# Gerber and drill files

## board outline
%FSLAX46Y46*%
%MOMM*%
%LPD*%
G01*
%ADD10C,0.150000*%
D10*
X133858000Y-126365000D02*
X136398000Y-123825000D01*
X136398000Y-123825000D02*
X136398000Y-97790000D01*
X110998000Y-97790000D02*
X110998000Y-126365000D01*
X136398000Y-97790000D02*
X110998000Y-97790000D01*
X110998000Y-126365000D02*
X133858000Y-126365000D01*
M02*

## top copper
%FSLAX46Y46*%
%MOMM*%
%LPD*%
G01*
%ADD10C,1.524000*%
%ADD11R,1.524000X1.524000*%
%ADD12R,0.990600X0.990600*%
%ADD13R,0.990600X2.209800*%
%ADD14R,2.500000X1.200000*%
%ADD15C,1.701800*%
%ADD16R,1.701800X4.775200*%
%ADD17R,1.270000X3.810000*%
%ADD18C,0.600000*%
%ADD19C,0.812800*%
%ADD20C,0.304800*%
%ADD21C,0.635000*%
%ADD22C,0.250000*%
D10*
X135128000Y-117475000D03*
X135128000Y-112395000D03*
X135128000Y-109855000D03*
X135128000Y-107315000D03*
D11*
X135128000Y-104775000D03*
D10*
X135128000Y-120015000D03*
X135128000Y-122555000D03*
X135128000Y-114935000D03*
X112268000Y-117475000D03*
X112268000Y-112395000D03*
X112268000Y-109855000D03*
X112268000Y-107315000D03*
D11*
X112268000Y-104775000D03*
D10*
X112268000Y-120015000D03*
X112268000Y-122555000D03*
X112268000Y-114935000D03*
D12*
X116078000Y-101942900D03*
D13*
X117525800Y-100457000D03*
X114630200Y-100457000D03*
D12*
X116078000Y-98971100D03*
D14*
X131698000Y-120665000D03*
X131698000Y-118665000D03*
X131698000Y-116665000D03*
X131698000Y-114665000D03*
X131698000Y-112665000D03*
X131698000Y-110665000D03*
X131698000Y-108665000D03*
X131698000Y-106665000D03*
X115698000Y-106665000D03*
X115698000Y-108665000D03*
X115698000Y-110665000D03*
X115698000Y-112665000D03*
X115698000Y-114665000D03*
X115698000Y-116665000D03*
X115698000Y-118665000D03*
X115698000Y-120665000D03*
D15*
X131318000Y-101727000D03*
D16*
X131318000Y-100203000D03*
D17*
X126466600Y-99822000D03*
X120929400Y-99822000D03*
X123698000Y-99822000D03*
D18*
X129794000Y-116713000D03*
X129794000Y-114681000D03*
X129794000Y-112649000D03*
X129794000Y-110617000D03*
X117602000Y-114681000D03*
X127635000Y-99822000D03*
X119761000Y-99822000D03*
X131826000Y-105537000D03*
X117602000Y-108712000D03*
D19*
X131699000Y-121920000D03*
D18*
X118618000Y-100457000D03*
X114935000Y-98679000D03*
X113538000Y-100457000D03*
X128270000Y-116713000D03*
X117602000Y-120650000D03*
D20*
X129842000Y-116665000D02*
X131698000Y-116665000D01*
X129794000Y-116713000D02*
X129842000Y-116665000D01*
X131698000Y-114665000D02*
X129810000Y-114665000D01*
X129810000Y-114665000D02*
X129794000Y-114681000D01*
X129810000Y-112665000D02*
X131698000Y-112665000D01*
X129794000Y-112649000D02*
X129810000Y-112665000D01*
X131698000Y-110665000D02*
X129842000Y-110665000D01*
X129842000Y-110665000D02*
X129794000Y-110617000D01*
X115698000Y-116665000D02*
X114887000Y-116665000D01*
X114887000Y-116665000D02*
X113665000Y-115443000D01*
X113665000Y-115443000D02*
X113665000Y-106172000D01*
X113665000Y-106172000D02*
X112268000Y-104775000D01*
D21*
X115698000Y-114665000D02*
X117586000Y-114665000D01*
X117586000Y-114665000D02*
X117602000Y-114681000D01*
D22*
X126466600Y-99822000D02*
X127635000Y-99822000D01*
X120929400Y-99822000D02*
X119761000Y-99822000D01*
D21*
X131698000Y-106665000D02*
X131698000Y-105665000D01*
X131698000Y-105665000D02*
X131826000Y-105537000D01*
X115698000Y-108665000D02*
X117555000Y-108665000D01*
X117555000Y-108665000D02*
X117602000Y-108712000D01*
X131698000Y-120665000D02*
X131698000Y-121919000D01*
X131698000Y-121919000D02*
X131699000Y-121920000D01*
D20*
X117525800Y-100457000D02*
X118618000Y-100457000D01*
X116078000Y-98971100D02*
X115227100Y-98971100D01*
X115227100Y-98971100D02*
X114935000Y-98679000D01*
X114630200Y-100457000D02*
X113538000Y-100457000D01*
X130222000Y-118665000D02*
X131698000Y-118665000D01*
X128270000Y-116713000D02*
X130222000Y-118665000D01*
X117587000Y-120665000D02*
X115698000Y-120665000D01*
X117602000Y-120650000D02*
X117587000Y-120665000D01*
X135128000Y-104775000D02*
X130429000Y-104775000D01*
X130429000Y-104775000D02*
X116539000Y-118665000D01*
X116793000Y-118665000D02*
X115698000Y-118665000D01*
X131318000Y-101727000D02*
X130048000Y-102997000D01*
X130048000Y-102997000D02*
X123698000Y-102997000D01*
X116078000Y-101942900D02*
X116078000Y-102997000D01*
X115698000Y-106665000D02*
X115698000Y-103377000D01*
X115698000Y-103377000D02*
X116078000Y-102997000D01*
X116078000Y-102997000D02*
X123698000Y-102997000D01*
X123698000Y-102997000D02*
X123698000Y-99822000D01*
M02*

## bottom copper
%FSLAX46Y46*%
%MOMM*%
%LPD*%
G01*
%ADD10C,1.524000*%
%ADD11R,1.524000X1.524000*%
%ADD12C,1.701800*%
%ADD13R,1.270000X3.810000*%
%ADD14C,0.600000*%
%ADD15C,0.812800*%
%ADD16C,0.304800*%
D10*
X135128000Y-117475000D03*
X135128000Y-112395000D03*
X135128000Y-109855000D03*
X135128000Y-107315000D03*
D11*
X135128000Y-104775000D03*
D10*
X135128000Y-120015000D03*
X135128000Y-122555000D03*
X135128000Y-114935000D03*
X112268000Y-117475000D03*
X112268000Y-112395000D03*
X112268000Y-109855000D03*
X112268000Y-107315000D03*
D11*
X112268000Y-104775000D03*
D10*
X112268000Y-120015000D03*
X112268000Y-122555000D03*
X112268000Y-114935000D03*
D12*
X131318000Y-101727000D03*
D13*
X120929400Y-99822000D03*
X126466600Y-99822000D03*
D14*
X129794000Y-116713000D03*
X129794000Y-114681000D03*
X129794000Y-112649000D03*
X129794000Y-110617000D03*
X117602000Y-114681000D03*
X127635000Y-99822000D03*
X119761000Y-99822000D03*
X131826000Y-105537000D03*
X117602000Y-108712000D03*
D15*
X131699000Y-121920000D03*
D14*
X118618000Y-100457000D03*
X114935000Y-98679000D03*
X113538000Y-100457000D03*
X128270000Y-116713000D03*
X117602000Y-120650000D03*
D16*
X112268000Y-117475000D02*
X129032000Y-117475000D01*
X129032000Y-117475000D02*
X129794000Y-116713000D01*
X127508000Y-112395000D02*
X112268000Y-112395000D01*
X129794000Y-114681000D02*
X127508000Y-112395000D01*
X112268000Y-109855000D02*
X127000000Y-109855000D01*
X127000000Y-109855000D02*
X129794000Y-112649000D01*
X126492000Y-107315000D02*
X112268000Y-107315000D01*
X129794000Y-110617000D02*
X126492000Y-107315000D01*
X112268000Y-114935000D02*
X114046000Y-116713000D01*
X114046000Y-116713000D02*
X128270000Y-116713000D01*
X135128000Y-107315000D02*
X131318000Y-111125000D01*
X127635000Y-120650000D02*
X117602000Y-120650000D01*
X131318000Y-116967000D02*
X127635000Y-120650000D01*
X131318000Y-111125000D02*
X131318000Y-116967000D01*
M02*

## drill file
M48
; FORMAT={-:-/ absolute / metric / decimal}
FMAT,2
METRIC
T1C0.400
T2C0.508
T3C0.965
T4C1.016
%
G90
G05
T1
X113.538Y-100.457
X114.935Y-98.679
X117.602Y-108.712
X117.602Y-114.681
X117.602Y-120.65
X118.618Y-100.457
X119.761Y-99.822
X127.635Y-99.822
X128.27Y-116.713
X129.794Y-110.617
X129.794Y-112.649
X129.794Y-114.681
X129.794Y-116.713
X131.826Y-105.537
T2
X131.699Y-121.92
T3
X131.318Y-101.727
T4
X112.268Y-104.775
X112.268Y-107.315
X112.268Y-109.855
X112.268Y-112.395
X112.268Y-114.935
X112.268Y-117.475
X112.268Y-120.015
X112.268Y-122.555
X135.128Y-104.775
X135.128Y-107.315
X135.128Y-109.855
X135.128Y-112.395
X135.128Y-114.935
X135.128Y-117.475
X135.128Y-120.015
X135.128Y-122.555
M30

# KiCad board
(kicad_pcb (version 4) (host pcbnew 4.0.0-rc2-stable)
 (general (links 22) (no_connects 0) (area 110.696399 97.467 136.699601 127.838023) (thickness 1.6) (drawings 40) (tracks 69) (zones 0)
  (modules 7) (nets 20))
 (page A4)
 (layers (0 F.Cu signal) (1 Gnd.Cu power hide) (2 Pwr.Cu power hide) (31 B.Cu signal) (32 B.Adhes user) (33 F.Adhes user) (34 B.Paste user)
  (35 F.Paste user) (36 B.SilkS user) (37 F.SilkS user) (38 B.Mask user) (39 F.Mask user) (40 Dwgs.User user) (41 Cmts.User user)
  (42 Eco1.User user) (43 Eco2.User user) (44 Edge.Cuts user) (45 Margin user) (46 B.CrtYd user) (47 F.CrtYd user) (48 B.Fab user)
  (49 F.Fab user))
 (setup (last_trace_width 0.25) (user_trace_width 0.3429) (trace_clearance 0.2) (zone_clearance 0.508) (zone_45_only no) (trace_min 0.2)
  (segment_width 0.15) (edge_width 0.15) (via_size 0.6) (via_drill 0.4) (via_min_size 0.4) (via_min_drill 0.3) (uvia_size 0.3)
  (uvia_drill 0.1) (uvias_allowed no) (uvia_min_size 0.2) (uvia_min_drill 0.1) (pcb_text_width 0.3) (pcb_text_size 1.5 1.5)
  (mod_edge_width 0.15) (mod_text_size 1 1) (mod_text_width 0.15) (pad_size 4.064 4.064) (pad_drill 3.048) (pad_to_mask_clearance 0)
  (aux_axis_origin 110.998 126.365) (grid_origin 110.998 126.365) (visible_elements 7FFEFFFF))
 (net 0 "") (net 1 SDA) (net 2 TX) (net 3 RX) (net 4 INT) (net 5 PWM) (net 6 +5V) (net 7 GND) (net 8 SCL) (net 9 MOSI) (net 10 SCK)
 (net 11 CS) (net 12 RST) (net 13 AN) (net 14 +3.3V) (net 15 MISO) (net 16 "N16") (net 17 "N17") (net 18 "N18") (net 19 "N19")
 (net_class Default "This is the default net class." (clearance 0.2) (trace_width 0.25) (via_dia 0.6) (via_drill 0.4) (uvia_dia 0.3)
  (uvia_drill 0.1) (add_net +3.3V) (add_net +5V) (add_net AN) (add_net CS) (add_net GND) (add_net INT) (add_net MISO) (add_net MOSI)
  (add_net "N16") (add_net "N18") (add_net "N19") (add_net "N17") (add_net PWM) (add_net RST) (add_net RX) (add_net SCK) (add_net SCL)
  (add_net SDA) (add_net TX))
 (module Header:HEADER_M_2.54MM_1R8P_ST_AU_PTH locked (layer B.Cu) (at 135.128 113.665 270)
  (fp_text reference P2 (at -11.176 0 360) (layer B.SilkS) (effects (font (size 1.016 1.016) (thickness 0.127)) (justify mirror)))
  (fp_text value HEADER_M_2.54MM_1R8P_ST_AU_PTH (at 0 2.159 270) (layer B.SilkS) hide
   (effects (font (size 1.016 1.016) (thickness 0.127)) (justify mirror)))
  (pad 6 thru_hole circle (at 3.81 0 270) (size 1.524 1.524) (drill 1.016) (layers *.Cu *.Mask) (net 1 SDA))
  (pad 4 thru_hole circle (at -1.27 0 270) (size 1.524 1.524) (drill 1.016) (layers *.Cu *.Mask) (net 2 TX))
  (pad 3 thru_hole circle (at -3.81 0 270) (size 1.524 1.524) (drill 1.016) (layers *.Cu *.Mask) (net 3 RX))
  (pad 2 thru_hole circle (at -6.35 0 270) (size 1.524 1.524) (drill 1.016) (layers *.Cu *.Mask) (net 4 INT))
  (pad 1 thru_hole rect (at -8.89 0 270) (size 1.524 1.524) (drill 1.016) (layers *.Cu *.Mask) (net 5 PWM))
  (pad 7 thru_hole circle (at 6.35 0 270) (size 1.524 1.524) (drill 1.016) (layers *.Cu *.Mask) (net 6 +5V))
  (pad 8 thru_hole circle (at 8.89 0 270) (size 1.524 1.524) (drill 1.016) (layers *.Cu *.Mask) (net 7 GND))
  (pad 5 thru_hole circle (at 1.27 0 270) (size 1.524 1.524) (drill 1.016) (layers *.Cu *.Mask) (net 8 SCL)))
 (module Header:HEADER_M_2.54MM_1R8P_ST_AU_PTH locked (layer B.Cu) (at 112.268 113.665 270)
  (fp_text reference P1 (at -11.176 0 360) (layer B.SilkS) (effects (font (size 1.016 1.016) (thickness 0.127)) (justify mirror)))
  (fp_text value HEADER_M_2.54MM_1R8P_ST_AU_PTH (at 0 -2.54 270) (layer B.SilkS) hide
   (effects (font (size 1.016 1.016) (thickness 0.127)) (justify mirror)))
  (pad 6 thru_hole circle (at 3.81 0 270) (size 1.524 1.524) (drill 1.016) (layers *.Cu *.Mask) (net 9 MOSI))
  (pad 4 thru_hole circle (at -1.27 0 270) (size 1.524 1.524) (drill 1.016) (layers *.Cu *.Mask) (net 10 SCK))
  (pad 3 thru_hole circle (at -3.81 0 270) (size 1.524 1.524) (drill 1.016) (layers *.Cu *.Mask) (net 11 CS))
  (pad 2 thru_hole circle (at -6.35 0 270) (size 1.524 1.524) (drill 1.016) (layers *.Cu *.Mask) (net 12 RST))
  (pad 1 thru_hole rect (at -8.89 0 270) (size 1.524 1.524) (drill 1.016) (layers *.Cu *.Mask) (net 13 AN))
  (pad 7 thru_hole circle (at 6.35 0 270) (size 1.524 1.524) (drill 1.016) (layers *.Cu *.Mask) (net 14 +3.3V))
  (pad 8 thru_hole circle (at 8.89 0 270) (size 1.524 1.524) (drill 1.016) (layers *.Cu *.Mask) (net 7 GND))
  (pad 5 thru_hole circle (at 1.27 0 270) (size 1.524 1.524) (drill 1.016) (layers *.Cu *.Mask) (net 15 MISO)))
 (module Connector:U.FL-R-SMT (layer F.Cu) (at 116.078 100.457)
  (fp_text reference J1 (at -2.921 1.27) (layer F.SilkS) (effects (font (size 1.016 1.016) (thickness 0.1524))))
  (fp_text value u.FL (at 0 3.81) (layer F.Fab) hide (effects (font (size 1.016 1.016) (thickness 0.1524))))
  (pad 1 smd rect (at 0 1.4859) (size 0.9906 0.9906) (layers F.Cu F.Paste F.Mask) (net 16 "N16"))
  (pad 4 smd rect (at 1.4478 0) (size 0.9906 2.2098) (layers F.Cu F.Paste F.Mask) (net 7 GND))
  (pad 2 smd rect (at -1.4478 0) (size 0.9906 2.2098) (layers F.Cu F.Paste F.Mask) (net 7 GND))
  (pad 3 smd rect (at 0 -1.4859) (size 0.9906 0.9906) (layers F.Cu F.Paste F.Mask) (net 7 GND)))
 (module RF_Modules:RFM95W (layer F.Cu) (at 123.698 113.665 180)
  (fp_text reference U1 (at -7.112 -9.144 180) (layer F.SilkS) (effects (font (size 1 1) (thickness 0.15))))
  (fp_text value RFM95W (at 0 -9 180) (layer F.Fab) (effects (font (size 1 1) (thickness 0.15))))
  (pad 1 smd rect (at -8 -7 180) (size 2.5 1.2) (layers F.Cu F.Paste F.Mask) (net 7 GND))
  (pad 2 smd rect (at -8 -5 180) (size 2.5 1.2) (layers F.Cu F.Paste F.Mask) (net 15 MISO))
  (pad 3 smd rect (at -8 -3 180) (size 2.5 1.2) (layers F.Cu F.Paste F.Mask) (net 9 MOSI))
  (pad 4 smd rect (at -8 -1 180) (size 2.5 1.2) (layers F.Cu F.Paste F.Mask) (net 10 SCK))
  (pad 5 smd rect (at -8 1 180) (size 2.5 1.2) (layers F.Cu F.Paste F.Mask) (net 11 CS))
  (pad 6 smd rect (at -8 3 180) (size 2.5 1.2) (layers F.Cu F.Paste F.Mask) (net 12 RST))
  (pad 7 smd rect (at -8 5 180) (size 2.5 1.2) (layers F.Cu F.Paste F.Mask) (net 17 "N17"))
  (pad 8 smd rect (at -8 7 180) (size 2.5 1.2) (layers F.Cu F.Paste F.Mask) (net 7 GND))
  (pad 9 smd rect (at 8 7 180) (size 2.5 1.2) (layers F.Cu F.Paste F.Mask) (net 16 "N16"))
  (pad 10 smd rect (at 8 5 180) (size 2.5 1.2) (layers F.Cu F.Paste F.Mask) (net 7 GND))
  (pad 11 smd rect (at 8 3 180) (size 2.5 1.2) (layers F.Cu F.Paste F.Mask) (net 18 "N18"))
  (pad 12 smd rect (at 8 1 180) (size 2.5 1.2) (layers F.Cu F.Paste F.Mask) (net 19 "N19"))
  (pad 13 smd rect (at 8 -1 180) (size 2.5 1.2) (layers F.Cu F.Paste F.Mask) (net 14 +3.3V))
  (pad 14 smd rect (at 8 -3 180) (size 2.5 1.2) (layers F.Cu F.Paste F.Mask) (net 13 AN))
  (pad 15 smd rect (at 8 -5 180) (size 2.5 1.2) (layers F.Cu F.Paste F.Mask) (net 5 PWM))
  (pad 16 smd rect (at 8 -7 180) (size 2.5 1.2) (layers F.Cu F.Paste F.Mask) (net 4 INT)))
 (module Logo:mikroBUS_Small (layer B.Cu) (at 123.698 104.775 180)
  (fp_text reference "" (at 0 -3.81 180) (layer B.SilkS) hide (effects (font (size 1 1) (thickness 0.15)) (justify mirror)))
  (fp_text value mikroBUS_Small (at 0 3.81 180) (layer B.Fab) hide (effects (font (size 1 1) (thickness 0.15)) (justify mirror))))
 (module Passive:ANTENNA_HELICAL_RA (layer F.Cu) (at 131.318 101.727)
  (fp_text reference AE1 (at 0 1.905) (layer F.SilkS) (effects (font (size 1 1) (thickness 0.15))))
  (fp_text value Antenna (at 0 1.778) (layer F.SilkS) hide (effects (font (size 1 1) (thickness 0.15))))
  (pad 1 thru_hole circle (at 0 0) (size 1.7018 1.7018) (drill 0.9652) (layers *.Cu *.Mask) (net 16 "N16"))
  (pad 1 smd rect (at 0 -1.524) (size 1.7018 4.7752) (layers F.Cu F.Mask) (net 16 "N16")))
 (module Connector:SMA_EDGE (layer F.Cu) (at 123.698 97.917 270)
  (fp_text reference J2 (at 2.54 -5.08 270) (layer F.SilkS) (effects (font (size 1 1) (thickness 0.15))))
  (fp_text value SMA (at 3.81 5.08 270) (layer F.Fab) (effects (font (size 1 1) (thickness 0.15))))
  (pad "" smd rect (at 1.905 2.7686 270) (size 3.81 1.27) (layers B.Cu))
  (pad "" smd rect (at 1.905 -2.7686 270) (size 3.81 1.27) (layers B.Cu))
  (pad 2 smd rect (at 1.905 -2.7686 270) (size 3.81 1.27) (layers F.Cu) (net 7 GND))
  (pad 3 smd rect (at 1.905 2.7686 270) (size 3.81 1.27) (layers F.Cu) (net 7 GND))
  (pad 1 smd rect (at 1.905 0 270) (size 3.81 1.27) (layers F.Cu F.Paste F.Mask) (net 16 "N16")))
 (gr_line (start 133.858 126.365) (end 136.398 123.825) (angle 90) (layer Edge.Cuts) (width 0.15))
 (gr_line (start 136.398 123.825) (end 136.398 97.79) (angle 90) (layer Edge.Cuts) (width 0.15))
 (gr_line (start 110.998 97.79) (end 110.998 126.365) (angle 90) (layer Edge.Cuts) (width 0.15))
 (gr_line (start 136.398 97.79) (end 110.998 97.79) (angle 90) (layer Edge.Cuts) (width 0.15))
 (gr_line (start 110.998 126.365) (end 133.858 126.365) (angle 90) (layer Edge.Cuts) (width 0.15))
 (segment (start 112.268 117.475) (end 129.032 117.475) (width 0.3048) (layer B.Cu) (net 9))
 (segment (start 129.842 116.665) (end 131.698 116.665) (width 0.3048) (layer F.Cu) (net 9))
 (segment (start 129.794 116.713) (end 129.842 116.665) (width 0.3048) (layer F.Cu) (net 9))
 (via (at 129.794 116.713) (size 0.6) (drill 0.4) (layers F.Cu B.Cu) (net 9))
 (segment (start 129.032 117.475) (end 129.794 116.713) (width 0.3048) (layer B.Cu) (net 9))
 (segment (start 131.698 114.665) (end 129.81 114.665) (width 0.3048) (layer F.Cu) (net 10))
 (segment (start 127.508 112.395) (end 112.268 112.395) (width 0.3048) (layer B.Cu) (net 10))
 (segment (start 129.794 114.681) (end 127.508 112.395) (width 0.3048) (layer B.Cu) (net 10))
 (via (at 129.794 114.681) (size 0.6) (drill 0.4) (layers F.Cu B.Cu) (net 10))
 (segment (start 129.81 114.665) (end 129.794 114.681) (width 0.3048) (layer F.Cu) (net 10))
 (segment (start 112.268 109.855) (end 127 109.855) (width 0.3048) (layer B.Cu) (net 11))
 (segment (start 129.81 112.665) (end 131.698 112.665) (width 0.3048) (layer F.Cu) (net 11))
 (segment (start 129.794 112.649) (end 129.81 112.665) (width 0.3048) (layer F.Cu) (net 11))
 (via (at 129.794 112.649) (size 0.6) (drill 0.4) (layers F.Cu B.Cu) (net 11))
 (segment (start 127 109.855) (end 129.794 112.649) (width 0.3048) (layer B.Cu) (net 11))
 (segment (start 131.698 110.665) (end 129.842 110.665) (width 0.3048) (layer F.Cu) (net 12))
 (segment (start 126.492 107.315) (end 112.268 107.315) (width 0.3048) (layer B.Cu) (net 12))
 (segment (start 129.794 110.617) (end 126.492 107.315) (width 0.3048) (layer B.Cu) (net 12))
 (via (at 129.794 110.617) (size 0.6) (drill 0.4) (layers F.Cu B.Cu) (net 12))
 (segment (start 129.842 110.665) (end 129.794 110.617) (width 0.3048) (layer F.Cu) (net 12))
 (segment (start 115.698 116.665) (end 114.887 116.665) (width 0.3048) (layer F.Cu) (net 13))
 (segment (start 114.887 116.665) (end 113.665 115.443) (width 0.3048) (layer F.Cu) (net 13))
 (segment (start 113.665 115.443) (end 113.665 106.172) (width 0.3048) (layer F.Cu) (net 13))
 (segment (start 113.665 106.172) (end 112.268 104.775) (width 0.3048) (layer F.Cu) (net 13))
 (segment (start 115.698 114.665) (end 117.586 114.665) (width 0.635) (layer F.Cu) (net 14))
 (via (at 117.602 114.681) (size 0.6) (drill 0.4) (layers F.Cu B.Cu) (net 14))
 (segment (start 117.586 114.665) (end 117.602 114.681) (width 0.635) (layer F.Cu) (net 14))
 (segment (start 126.4666 99.822) (end 127.635 99.822) (width 0.25) (layer F.Cu) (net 7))
 (via (at 127.635 99.822) (size 0.6) (drill 0.4) (layers F.Cu B.Cu) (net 7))
 (segment (start 120.9294 99.822) (end 119.761 99.822) (width 0.25) (layer F.Cu) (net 7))
 (via (at 119.761 99.822) (size 0.6) (drill 0.4) (layers F.Cu B.Cu) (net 7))
 (segment (start 131.698 106.665) (end 131.698 105.665) (width 0.635) (layer F.Cu) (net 7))
 (via (at 131.826 105.537) (size 0.6) (drill 0.4) (layers F.Cu B.Cu) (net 7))
 (segment (start 131.698 105.665) (end 131.826 105.537) (width 0.635) (layer F.Cu) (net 7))
 (segment (start 115.698 108.665) (end 117.555 108.665) (width 0.635) (layer F.Cu) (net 7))
 (via (at 117.602 108.712) (size 0.6) (drill 0.4) (layers F.Cu B.Cu) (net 7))
 (segment (start 117.555 108.665) (end 117.602 108.712) (width 0.635) (layer F.Cu) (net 7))
 (segment (start 131.698 120.665) (end 131.698 121.919) (width 0.635) (layer F.Cu) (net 7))
 (via (at 131.699 121.92) (size 0.8128) (drill 0.508) (layers F.Cu B.Cu) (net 7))
 (segment (start 131.698 121.919) (end 131.699 121.92) (width 0.635) (layer F.Cu) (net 7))
 (segment (start 117.5258 100.457) (end 118.618 100.457) (width 0.3048) (layer F.Cu) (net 7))
 (via (at 118.618 100.457) (size 0.6) (drill 0.4) (layers F.Cu B.Cu) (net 7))
 (segment (start 116.078 98.9711) (end 115.2271 98.9711) (width 0.3048) (layer F.Cu) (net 7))
 (via (at 114.935 98.679) (size 0.6) (drill 0.4) (layers F.Cu B.Cu) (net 7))
 (segment (start 115.2271 98.9711) (end 114.935 98.679) (width 0.3048) (layer F.Cu) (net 7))
 (segment (start 114.6302 100.457) (end 113.538 100.457) (width 0.3048) (layer F.Cu) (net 7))
 (via (at 113.538 100.457) (size 0.6) (drill 0.4) (layers F.Cu B.Cu) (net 7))
 (segment (start 112.268 114.935) (end 114.046 116.713) (width 0.3048) (layer B.Cu) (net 15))
 (segment (start 130.222 118.665) (end 131.698 118.665) (width 0.3048) (layer F.Cu) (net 15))
 (segment (start 128.27 116.713) (end 130.222 118.665) (width 0.3048) (layer F.Cu) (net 15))
 (via (at 128.27 116.713) (size 0.6) (drill 0.4) (layers F.Cu B.Cu) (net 15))
 (segment (start 114.046 116.713) (end 128.27 116.713) (width 0.3048) (layer B.Cu) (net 15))
 (segment (start 135.128 107.315) (end 131.318 111.125) (width 0.3048) (layer B.Cu) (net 4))
 (segment (start 117.587 120.665) (end 115.698 120.665) (width 0.3048) (layer F.Cu) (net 4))
 (segment (start 117.602 120.65) (end 117.587 120.665) (width 0.3048) (layer F.Cu) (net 4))
 (via (at 117.602 120.65) (size 0.6) (drill 0.4) (layers F.Cu B.Cu) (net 4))
 (segment (start 127.635 120.65) (end 117.602 120.65) (width 0.3048) (layer B.Cu) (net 4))
 (segment (start 131.318 116.967) (end 127.635 120.65) (width 0.3048) (layer B.Cu) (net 4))
 (segment (start 131.318 111.125) (end 131.318 116.967) (width 0.3048) (layer B.Cu) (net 4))
 (segment (start 135.128 104.775) (end 130.429 104.775) (width 0.3048) (layer F.Cu) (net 5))
 (segment (start 130.429 104.775) (end 116.539 118.665) (width 0.3048) (layer F.Cu) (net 5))
 (segment (start 116.793 118.665) (end 115.698 118.665) (width 0.3048) (layer F.Cu) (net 5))
 (segment (start 131.318 101.727) (end 130.048 102.997) (width 0.3048) (layer F.Cu) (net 16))
 (segment (start 130.048 102.997) (end 123.698 102.997) (width 0.3048) (layer F.Cu) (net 16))
 (segment (start 116.078 101.9429) (end 116.078 102.997) (width 0.3048) (layer F.Cu) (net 16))
 (segment (start 115.698 106.665) (end 115.698 103.377) (width 0.3048) (layer F.Cu) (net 16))
 (segment (start 115.698 103.377) (end 116.078 102.997) (width 0.3048) (layer F.Cu) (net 16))
 (segment (start 116.078 102.997) (end 123.698 102.997) (width 0.3048) (layer F.Cu) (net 16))
 (segment (start 123.698 102.997) (end 123.698 99.822) (width 0.3048) (layer F.Cu) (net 16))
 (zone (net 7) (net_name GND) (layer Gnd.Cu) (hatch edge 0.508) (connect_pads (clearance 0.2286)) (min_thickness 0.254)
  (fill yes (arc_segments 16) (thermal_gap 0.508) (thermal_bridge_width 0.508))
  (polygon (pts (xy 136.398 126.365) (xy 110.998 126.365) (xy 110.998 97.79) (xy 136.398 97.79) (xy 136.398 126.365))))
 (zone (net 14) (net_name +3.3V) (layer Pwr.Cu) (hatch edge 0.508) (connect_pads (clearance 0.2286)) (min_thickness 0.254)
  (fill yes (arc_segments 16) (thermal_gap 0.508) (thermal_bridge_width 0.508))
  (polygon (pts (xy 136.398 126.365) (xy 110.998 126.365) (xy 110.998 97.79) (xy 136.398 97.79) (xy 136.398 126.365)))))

